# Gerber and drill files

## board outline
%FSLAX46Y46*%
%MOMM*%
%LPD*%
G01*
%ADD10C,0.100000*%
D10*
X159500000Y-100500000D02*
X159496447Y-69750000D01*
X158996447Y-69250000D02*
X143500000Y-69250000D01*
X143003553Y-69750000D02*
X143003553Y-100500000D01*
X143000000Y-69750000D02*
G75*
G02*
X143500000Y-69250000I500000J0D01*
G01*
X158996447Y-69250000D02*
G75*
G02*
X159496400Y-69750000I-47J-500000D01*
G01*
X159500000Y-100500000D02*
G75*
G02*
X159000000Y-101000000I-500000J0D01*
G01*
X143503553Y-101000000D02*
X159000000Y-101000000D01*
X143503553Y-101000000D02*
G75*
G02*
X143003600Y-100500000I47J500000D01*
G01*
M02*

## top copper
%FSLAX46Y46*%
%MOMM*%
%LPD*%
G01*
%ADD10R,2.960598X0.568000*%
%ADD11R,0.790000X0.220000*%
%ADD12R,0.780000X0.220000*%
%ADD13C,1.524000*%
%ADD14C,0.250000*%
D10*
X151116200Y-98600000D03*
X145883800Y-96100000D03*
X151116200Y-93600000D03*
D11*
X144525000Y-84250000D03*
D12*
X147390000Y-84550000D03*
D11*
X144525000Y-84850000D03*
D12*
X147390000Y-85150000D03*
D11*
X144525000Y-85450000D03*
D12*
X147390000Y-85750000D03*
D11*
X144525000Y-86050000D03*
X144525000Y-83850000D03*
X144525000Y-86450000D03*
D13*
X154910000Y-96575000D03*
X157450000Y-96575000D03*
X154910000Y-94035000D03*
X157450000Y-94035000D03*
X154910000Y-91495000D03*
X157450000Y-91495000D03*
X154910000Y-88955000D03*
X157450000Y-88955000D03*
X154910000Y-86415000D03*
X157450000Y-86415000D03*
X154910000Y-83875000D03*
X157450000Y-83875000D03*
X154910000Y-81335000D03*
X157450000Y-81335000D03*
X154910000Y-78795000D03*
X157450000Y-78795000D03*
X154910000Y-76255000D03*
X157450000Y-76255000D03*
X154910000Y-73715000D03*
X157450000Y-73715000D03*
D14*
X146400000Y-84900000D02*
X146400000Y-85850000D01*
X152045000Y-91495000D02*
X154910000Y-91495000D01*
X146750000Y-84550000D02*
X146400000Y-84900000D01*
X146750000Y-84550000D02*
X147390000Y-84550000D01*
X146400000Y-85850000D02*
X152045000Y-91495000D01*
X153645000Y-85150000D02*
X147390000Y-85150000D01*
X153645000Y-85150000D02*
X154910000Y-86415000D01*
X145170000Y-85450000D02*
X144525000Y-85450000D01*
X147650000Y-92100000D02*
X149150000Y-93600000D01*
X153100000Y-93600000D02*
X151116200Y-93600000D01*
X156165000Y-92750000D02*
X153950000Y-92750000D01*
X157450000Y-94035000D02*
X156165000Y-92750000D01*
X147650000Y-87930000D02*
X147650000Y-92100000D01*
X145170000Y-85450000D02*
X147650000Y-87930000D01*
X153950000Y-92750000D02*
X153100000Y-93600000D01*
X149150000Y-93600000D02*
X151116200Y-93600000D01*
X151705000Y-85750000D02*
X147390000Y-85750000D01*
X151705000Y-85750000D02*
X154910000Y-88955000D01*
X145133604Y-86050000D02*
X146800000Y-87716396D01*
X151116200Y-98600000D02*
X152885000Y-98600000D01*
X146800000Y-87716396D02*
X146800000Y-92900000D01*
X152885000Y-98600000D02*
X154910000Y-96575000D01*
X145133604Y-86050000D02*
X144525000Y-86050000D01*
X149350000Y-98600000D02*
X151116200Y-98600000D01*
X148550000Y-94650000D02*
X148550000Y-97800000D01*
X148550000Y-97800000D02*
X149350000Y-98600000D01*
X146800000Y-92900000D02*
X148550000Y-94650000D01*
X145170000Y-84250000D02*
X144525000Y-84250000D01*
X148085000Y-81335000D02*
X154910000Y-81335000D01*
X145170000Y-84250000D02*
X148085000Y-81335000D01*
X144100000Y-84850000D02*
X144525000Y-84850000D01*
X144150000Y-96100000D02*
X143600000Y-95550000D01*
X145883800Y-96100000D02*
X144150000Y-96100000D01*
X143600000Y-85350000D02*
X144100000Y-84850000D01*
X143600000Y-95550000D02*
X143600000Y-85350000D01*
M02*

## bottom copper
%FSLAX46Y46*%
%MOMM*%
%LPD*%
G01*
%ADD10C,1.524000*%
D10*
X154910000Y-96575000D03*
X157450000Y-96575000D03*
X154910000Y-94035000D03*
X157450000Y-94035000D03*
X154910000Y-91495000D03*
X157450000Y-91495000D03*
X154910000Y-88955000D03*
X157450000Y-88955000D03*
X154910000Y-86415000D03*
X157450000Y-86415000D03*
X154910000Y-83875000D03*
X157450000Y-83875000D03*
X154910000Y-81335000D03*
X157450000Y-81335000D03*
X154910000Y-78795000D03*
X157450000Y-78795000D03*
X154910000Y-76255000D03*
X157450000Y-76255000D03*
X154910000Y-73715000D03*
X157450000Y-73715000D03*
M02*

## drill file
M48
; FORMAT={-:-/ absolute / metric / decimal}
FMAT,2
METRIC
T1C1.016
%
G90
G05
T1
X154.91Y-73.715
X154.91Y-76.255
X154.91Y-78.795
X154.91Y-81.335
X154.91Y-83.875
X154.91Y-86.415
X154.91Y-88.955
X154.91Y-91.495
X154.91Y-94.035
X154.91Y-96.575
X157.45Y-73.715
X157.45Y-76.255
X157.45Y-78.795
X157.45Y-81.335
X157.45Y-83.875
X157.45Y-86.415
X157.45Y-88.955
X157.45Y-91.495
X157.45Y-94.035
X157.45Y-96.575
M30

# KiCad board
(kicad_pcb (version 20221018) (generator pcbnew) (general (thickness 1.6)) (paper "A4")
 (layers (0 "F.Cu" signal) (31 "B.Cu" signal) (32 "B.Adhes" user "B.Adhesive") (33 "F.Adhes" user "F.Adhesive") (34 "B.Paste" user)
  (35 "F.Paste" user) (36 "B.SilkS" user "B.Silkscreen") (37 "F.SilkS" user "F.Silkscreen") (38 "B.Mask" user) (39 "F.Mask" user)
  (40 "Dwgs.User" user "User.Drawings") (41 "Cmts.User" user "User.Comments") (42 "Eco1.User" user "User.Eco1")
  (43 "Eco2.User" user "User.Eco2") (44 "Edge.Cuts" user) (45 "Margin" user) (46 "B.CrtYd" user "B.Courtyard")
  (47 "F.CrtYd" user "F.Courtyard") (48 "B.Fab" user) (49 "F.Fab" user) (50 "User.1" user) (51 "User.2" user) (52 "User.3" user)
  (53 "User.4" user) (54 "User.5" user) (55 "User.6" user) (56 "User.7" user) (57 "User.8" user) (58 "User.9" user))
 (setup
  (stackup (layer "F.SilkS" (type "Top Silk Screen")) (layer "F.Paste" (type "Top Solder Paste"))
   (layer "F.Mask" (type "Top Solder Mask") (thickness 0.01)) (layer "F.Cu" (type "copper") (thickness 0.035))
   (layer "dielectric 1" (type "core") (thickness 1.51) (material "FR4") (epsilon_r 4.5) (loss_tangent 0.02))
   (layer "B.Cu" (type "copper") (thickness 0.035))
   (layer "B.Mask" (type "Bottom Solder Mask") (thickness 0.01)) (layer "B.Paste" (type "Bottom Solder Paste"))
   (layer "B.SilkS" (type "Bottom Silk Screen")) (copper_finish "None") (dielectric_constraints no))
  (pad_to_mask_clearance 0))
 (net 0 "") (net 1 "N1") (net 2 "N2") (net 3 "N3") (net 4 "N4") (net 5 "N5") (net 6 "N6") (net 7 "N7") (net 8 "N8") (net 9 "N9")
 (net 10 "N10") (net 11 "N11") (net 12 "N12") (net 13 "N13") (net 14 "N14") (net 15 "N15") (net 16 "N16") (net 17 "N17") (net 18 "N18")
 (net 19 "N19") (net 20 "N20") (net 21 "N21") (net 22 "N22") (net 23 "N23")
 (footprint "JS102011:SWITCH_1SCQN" (layer "F.Cu") (at 148.5 96.1 180)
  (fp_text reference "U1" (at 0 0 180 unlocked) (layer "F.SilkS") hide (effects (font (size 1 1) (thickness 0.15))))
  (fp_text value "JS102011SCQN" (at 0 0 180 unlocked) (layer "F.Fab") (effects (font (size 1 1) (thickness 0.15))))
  (pad "1" smd rect (at -2.6162 -2.5 180) (size 2.960598 0.568) (layers "F.Cu" "F.Paste" "F.Mask") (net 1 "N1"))
  (pad "2" smd rect (at 2.6162 0 180) (size 2.960598 0.568) (layers "F.Cu" "F.Paste" "F.Mask") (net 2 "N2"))
  (pad "3" smd rect (at -2.6162 2.5 180) (size 2.960598 0.568) (layers "F.Cu" "F.Paste" "F.Mask") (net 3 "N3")))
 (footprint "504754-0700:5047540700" (layer "F.Cu") (at 145.98 85.15 -90)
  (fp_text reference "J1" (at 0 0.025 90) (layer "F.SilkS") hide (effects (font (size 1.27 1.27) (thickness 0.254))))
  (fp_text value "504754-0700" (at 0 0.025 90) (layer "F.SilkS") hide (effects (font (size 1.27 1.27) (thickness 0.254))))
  (pad "1" smd rect (at -0.9 1.455 270) (size 0.22 0.79) (layers "F.Cu" "F.Paste" "F.Mask") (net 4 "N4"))
  (pad "2" smd rect (at -0.6 -1.41 270) (size 0.22 0.78) (layers "F.Cu" "F.Paste" "F.Mask") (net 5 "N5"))
  (pad "3" smd rect (at -0.3 1.455 270) (size 0.22 0.79) (layers "F.Cu" "F.Paste" "F.Mask") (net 2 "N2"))
  (pad "4" smd rect (at 0 -1.41 270) (size 0.22 0.78) (layers "F.Cu" "F.Paste" "F.Mask") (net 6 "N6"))
  (pad "5" smd rect (at 0.3 1.455 270) (size 0.22 0.79) (layers "F.Cu" "F.Paste" "F.Mask") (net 3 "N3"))
  (pad "6" smd rect (at 0.6 -1.41 270) (size 0.22 0.78) (layers "F.Cu" "F.Paste" "F.Mask") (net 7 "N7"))
  (pad "7" smd rect (at 0.9 1.455 270) (size 0.22 0.79) (layers "F.Cu" "F.Paste" "F.Mask") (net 1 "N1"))
  (pad "MP1" smd rect (at -1.3 1.455 270) (size 0.22 0.79) (layers "F.Cu" "F.Paste" "F.Mask") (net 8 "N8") (clearance 0.001))
  (pad "MP2" smd rect (at 1.3 1.455 270) (size 0.22 0.79) (layers "F.Cu" "F.Paste" "F.Mask") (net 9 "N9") (clearance 0.001)))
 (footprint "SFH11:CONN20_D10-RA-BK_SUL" (layer "F.Cu") (at 154.91 96.575 90)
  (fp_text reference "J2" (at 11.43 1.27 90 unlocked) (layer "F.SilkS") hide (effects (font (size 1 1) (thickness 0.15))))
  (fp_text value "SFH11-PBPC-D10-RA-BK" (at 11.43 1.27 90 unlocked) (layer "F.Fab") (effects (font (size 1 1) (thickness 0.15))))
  (pad "1" thru_hole circle (at 0 0 90) (size 1.524 1.524) (drill 1.016) (layers "*.Cu" "*.Mask") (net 1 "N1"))
  (pad "2" thru_hole circle (at 0 2.54 90) (size 1.524 1.524) (drill 1.016) (layers "*.Cu" "*.Mask") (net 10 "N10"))
  (pad "3" thru_hole circle (at 2.54 0 90) (size 1.524 1.524) (drill 1.016) (layers "*.Cu" "*.Mask") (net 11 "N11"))
  (pad "4" thru_hole circle (at 2.54 2.54 90) (size 1.524 1.524) (drill 1.016) (layers "*.Cu" "*.Mask") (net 3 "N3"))
  (pad "5" thru_hole circle (at 5.08 0 90) (size 1.524 1.524) (drill 1.016) (layers "*.Cu" "*.Mask") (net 5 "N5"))
  (pad "6" thru_hole circle (at 5.08 2.54 90) (size 1.524 1.524) (drill 1.016) (layers "*.Cu" "*.Mask") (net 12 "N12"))
  (pad "7" thru_hole circle (at 7.62 0 90) (size 1.524 1.524) (drill 1.016) (layers "*.Cu" "*.Mask") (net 7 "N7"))
  (pad "8" thru_hole circle (at 7.62 2.54 90) (size 1.524 1.524) (drill 1.016) (layers "*.Cu" "*.Mask") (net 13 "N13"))
  (pad "9" thru_hole circle (at 10.16 0 90) (size 1.524 1.524) (drill 1.016) (layers "*.Cu" "*.Mask") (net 6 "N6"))
  (pad "10" thru_hole circle (at 10.16 2.54 90) (size 1.524 1.524) (drill 1.016) (layers "*.Cu" "*.Mask") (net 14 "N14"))
  (pad "11" thru_hole circle (at 12.7 0 90) (size 1.524 1.524) (drill 1.016) (layers "*.Cu" "*.Mask") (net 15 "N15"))
  (pad "12" thru_hole circle (at 12.7 2.54 90) (size 1.524 1.524) (drill 1.016) (layers "*.Cu" "*.Mask") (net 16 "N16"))
  (pad "13" thru_hole circle (at 15.24 0 90) (size 1.524 1.524) (drill 1.016) (layers "*.Cu" "*.Mask") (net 4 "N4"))
  (pad "14" thru_hole circle (at 15.24 2.54 90) (size 1.524 1.524) (drill 1.016) (layers "*.Cu" "*.Mask") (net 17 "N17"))
  (pad "15" thru_hole circle (at 17.78 0 90) (size 1.524 1.524) (drill 1.016) (layers "*.Cu" "*.Mask") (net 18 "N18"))
  (pad "16" thru_hole circle (at 17.78 2.54 90) (size 1.524 1.524) (drill 1.016) (layers "*.Cu" "*.Mask") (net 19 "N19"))
  (pad "17" thru_hole circle (at 20.32 0 90) (size 1.524 1.524) (drill 1.016) (layers "*.Cu" "*.Mask") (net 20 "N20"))
  (pad "18" thru_hole circle (at 20.32 2.54 90) (size 1.524 1.524) (drill 1.016) (layers "*.Cu" "*.Mask") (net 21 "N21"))
  (pad "19" thru_hole circle (at 22.86 0 90) (size 1.524 1.524) (drill 1.016) (layers "*.Cu" "*.Mask") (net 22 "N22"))
  (pad "20" thru_hole circle (at 22.86 2.54 90) (size 1.524 1.524) (drill 1.016) (layers "*.Cu" "*.Mask") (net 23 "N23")))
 (gr_line (start 159.5 100.5) (end 159.496447 69.75) (stroke (width 0.1) (type default)) (layer "Edge.Cuts"))
 (gr_line (start 158.996447 69.25) (end 143.5 69.25) (stroke (width 0.1) (type default)) (layer "Edge.Cuts"))
 (gr_line (start 143.003553 69.75) (end 143.003553 100.5) (stroke (width 0.1) (type default)) (layer "Edge.Cuts"))
 (gr_arc (start 143 69.75) (mid 143.146447 69.396447) (end 143.5 69.25) (stroke (width 0.1) (type default)) (layer "Edge.Cuts"))
 (gr_arc (start 158.996447 69.25) (mid 159.35 69.396447) (end 159.496447 69.75) (stroke (width 0.1) (type default)) (layer "Edge.Cuts"))
 (gr_arc (start 159.5 100.5) (mid 159.353553 100.853553) (end 159 101) (stroke (width 0.1) (type default)) (layer "Edge.Cuts"))
 (gr_line (start 143.503553 101) (end 159 101) (stroke (width 0.1) (type default)) (layer "Edge.Cuts"))
 (gr_arc (start 143.503553 101) (mid 143.15 100.853553) (end 143.003553 100.5) (stroke (width 0.1) (type default)) (layer "Edge.Cuts"))
 (segment (start 146.4 84.9) (end 146.4 85.85) (width 0.25) (layer "F.Cu") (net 5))
 (segment (start 152.045 91.495) (end 154.91 91.495) (width 0.25) (layer "F.Cu") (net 5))
 (segment (start 146.75 84.55) (end 146.4 84.9) (width 0.25) (layer "F.Cu") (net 5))
 (segment (start 146.75 84.55) (end 147.39 84.55) (width 0.25) (layer "F.Cu") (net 5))
 (segment (start 146.4 85.85) (end 152.045 91.495) (width 0.25) (layer "F.Cu") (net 5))
 (segment (start 153.645 85.15) (end 147.39 85.15) (width 0.25) (layer "F.Cu") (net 6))
 (segment (start 153.645 85.15) (end 154.91 86.415) (width 0.25) (layer "F.Cu") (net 6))
 (segment (start 145.17 85.45) (end 144.525 85.45) (width 0.25) (layer "F.Cu") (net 3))
 (segment (start 147.65 92.1) (end 149.15 93.6) (width 0.25) (layer "F.Cu") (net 3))
 (segment (start 153.1 93.6) (end 151.1162 93.6) (width 0.25) (layer "F.Cu") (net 3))
 (segment (start 156.165 92.75) (end 153.95 92.75) (width 0.25) (layer "F.Cu") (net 3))
 (segment (start 157.45 94.035) (end 156.165 92.75) (width 0.25) (layer "F.Cu") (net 3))
 (segment (start 147.65 87.93) (end 147.65 92.1) (width 0.25) (layer "F.Cu") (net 3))
 (segment (start 145.17 85.45) (end 147.65 87.93) (width 0.25) (layer "F.Cu") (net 3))
 (segment (start 153.95 92.75) (end 153.1 93.6) (width 0.25) (layer "F.Cu") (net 3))
 (segment (start 149.15 93.6) (end 151.1162 93.6) (width 0.25) (layer "F.Cu") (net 3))
 (segment (start 151.705 85.75) (end 147.39 85.75) (width 0.25) (layer "F.Cu") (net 7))
 (segment (start 151.705 85.75) (end 154.91 88.955) (width 0.25) (layer "F.Cu") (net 7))
 (segment (start 145.133604 86.05) (end 146.8 87.716396) (width 0.25) (layer "F.Cu") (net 1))
 (segment (start 151.1162 98.6) (end 152.885 98.6) (width 0.25) (layer "F.Cu") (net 1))
 (segment (start 146.8 87.716396) (end 146.8 92.9) (width 0.25) (layer "F.Cu") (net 1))
 (segment (start 152.885 98.6) (end 154.91 96.575) (width 0.25) (layer "F.Cu") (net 1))
 (segment (start 145.133604 86.05) (end 144.525 86.05) (width 0.25) (layer "F.Cu") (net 1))
 (segment (start 149.35 98.6) (end 151.1162 98.6) (width 0.25) (layer "F.Cu") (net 1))
 (segment (start 148.55 94.65) (end 148.55 97.8) (width 0.25) (layer "F.Cu") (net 1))
 (segment (start 148.55 97.8) (end 149.35 98.6) (width 0.25) (layer "F.Cu") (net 1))
 (segment (start 146.8 92.9) (end 148.55 94.65) (width 0.25) (layer "F.Cu") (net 1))
 (segment (start 145.17 84.25) (end 144.525 84.25) (width 0.25) (layer "F.Cu") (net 4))
 (segment (start 148.085 81.335) (end 154.91 81.335) (width 0.25) (layer "F.Cu") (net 4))
 (segment (start 145.17 84.25) (end 148.085 81.335) (width 0.25) (layer "F.Cu") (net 4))
 (segment (start 144.1 84.85) (end 144.525 84.85) (width 0.25) (layer "F.Cu") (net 2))
 (segment (start 144.15 96.1) (end 143.6 95.55) (width 0.25) (layer "F.Cu") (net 2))
 (segment (start 145.8838 96.1) (end 144.15 96.1) (width 0.25) (layer "F.Cu") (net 2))
 (segment (start 143.6 85.35) (end 144.1 84.85) (width 0.25) (layer "F.Cu") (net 2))
 (segment (start 143.6 95.55) (end 143.6 85.35) (width 0.25) (layer "F.Cu") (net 2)))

